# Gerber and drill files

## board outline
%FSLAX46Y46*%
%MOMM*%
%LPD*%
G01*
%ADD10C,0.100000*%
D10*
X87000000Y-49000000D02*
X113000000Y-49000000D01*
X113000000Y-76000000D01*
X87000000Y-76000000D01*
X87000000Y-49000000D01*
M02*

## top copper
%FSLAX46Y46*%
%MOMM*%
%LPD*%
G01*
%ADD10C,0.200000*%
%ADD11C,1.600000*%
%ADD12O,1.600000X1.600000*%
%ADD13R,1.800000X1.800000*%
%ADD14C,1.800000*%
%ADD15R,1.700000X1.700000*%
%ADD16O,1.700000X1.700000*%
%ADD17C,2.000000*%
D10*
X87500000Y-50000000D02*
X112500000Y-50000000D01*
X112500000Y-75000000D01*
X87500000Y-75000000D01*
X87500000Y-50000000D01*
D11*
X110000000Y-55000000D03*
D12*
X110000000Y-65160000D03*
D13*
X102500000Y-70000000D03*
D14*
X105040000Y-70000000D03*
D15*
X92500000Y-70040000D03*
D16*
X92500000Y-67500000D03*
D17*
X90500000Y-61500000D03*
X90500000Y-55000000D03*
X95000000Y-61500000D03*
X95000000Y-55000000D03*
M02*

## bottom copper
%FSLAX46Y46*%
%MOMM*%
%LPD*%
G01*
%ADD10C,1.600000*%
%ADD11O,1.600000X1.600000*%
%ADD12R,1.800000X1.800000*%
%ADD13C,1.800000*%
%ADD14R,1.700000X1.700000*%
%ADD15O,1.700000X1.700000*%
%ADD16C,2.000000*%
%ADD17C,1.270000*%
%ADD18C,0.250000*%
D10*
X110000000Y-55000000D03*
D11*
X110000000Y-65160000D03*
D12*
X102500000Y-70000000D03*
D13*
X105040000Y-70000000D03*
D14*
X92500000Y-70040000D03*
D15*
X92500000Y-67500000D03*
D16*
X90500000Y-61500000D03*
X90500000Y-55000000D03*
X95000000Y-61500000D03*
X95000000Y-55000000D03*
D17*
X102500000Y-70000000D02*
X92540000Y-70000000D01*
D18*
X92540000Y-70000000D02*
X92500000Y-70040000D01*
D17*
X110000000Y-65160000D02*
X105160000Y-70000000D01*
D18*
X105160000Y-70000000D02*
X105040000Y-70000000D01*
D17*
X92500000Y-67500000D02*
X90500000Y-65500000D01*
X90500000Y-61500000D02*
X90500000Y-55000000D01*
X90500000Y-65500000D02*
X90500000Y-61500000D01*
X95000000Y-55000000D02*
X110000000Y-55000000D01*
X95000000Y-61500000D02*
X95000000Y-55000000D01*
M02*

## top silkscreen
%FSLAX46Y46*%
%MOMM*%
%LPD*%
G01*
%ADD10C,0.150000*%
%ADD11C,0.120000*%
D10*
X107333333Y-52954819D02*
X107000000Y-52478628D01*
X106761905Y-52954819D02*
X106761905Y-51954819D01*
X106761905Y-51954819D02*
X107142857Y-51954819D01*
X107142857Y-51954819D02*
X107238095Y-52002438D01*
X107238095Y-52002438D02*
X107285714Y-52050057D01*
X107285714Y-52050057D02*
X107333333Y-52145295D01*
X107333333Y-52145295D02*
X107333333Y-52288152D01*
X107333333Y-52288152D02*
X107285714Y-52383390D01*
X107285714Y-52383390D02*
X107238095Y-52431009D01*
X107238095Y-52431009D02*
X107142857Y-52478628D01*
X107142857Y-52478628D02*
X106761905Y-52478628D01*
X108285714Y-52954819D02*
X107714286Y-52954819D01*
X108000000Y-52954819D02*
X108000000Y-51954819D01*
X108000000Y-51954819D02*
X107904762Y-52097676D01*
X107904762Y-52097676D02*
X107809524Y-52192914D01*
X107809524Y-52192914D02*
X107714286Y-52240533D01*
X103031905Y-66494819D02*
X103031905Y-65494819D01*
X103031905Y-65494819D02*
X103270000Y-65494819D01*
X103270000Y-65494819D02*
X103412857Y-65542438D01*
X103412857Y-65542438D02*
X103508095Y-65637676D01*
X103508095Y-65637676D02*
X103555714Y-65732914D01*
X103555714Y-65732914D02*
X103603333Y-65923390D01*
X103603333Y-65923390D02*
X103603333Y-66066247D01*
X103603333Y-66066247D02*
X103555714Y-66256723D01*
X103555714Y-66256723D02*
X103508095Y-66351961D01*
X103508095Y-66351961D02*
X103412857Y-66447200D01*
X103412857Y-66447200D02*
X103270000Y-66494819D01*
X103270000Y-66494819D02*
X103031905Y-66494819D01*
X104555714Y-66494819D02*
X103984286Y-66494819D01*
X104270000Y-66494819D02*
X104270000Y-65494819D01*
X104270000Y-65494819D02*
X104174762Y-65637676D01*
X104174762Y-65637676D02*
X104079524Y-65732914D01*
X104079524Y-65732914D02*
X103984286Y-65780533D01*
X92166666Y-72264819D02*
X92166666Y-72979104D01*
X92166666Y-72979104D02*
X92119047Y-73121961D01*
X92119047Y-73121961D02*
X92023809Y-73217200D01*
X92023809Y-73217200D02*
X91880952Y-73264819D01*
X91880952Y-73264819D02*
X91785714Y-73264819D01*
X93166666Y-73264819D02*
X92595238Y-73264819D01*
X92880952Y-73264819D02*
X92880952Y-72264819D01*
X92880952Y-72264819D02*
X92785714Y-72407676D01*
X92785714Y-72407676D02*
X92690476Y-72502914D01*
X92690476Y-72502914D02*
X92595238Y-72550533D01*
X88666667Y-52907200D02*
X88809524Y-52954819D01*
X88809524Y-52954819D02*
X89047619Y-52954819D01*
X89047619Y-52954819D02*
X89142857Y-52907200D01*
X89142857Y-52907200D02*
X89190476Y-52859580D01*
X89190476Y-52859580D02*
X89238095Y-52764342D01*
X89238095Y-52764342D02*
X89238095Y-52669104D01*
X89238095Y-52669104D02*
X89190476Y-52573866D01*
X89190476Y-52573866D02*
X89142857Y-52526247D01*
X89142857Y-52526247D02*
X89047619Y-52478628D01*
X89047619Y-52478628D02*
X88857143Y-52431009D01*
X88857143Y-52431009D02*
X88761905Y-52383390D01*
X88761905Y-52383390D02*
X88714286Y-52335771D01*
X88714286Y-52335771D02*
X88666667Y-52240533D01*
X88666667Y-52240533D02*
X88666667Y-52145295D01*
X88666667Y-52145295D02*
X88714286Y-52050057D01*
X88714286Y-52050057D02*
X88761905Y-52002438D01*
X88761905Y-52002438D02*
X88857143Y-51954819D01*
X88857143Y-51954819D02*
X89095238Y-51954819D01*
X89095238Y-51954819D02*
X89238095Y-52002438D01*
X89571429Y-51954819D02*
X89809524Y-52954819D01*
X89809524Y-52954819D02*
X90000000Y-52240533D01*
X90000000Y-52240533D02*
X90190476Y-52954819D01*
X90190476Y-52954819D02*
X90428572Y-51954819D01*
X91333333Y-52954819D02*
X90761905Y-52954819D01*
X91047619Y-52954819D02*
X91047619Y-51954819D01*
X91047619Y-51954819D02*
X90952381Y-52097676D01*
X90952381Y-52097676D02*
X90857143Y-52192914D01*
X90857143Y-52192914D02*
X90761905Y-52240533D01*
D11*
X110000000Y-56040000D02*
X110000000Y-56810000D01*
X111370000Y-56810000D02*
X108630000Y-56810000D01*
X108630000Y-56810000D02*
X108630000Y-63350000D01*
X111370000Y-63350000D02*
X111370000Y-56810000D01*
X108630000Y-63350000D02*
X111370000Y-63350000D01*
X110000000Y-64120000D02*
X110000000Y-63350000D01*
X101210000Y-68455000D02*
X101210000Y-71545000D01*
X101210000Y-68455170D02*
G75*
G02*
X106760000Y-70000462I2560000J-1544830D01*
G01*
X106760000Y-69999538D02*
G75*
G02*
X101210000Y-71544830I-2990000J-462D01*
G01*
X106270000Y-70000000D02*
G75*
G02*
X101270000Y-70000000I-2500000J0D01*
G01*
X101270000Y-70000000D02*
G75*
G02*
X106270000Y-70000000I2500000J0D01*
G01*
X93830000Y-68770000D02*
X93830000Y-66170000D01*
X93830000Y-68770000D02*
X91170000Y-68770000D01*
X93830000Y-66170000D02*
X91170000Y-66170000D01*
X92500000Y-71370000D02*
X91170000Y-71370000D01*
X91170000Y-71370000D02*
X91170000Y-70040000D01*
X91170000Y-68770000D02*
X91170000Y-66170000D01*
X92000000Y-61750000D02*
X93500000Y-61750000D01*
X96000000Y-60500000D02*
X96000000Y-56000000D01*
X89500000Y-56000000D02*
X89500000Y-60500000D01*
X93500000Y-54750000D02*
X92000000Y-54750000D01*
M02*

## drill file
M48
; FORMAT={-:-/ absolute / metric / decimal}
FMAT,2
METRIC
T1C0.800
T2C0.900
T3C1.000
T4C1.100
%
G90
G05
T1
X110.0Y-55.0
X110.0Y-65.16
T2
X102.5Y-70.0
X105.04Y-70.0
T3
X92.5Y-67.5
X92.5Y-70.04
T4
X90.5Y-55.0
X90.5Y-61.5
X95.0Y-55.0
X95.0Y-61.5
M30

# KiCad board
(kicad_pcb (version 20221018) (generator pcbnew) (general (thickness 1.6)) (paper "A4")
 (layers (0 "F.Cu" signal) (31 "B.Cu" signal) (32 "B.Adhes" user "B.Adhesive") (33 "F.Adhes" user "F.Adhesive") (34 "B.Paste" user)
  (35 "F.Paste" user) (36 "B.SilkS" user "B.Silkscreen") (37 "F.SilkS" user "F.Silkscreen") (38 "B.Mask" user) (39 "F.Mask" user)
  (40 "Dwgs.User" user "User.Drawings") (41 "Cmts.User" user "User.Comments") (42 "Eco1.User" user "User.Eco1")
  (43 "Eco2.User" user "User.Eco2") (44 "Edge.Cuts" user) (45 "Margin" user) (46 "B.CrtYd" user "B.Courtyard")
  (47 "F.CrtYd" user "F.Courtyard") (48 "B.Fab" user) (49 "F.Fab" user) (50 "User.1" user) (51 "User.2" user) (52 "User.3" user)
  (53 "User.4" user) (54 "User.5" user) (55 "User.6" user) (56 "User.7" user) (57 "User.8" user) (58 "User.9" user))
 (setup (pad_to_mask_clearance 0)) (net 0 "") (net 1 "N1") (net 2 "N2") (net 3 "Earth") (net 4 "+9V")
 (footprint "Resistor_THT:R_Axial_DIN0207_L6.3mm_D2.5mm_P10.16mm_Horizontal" (layer "F.Cu") (at 110 55 -90)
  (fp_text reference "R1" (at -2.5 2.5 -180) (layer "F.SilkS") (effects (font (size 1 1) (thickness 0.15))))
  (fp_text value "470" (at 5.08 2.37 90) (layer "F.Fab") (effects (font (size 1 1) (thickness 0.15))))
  (fp_line (start 1.04 0) (end 1.81 0) (stroke (width 0.12) (type solid)) (layer "F.SilkS"))
  (fp_line (start 1.81 -1.37) (end 1.81 1.37) (stroke (width 0.12) (type solid)) (layer "F.SilkS"))
  (fp_line (start 1.81 1.37) (end 8.35 1.37) (stroke (width 0.12) (type solid)) (layer "F.SilkS"))
  (fp_line (start 8.35 -1.37) (end 1.81 -1.37) (stroke (width 0.12) (type solid)) (layer "F.SilkS"))
  (fp_line (start 8.35 1.37) (end 8.35 -1.37) (stroke (width 0.12) (type solid)) (layer "F.SilkS"))
  (fp_line (start 9.12 0) (end 8.35 0) (stroke (width 0.12) (type solid)) (layer "F.SilkS"))
  (pad "1" thru_hole circle (at 0 0 270) (size 1.6 1.6) (drill 0.8) (layers "*.Cu" "*.Mask") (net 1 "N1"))
  (pad "2" thru_hole oval (at 10.16 0 270) (size 1.6 1.6) (drill 0.8) (layers "*.Cu" "*.Mask") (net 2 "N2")))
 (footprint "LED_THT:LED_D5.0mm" (layer "F.Cu") (at 102.5 70)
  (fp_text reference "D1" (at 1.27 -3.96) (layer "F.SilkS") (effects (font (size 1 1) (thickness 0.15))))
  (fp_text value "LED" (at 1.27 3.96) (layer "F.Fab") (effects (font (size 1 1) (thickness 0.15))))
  (fp_line (start -1.29 -1.545) (end -1.29 1.545) (stroke (width 0.12) (type solid)) (layer "F.SilkS"))
  (fp_arc (start -1.29 -1.54483) (mid 2.072002 -2.880433) (end 4.26 0.000462) (stroke (width 0.12) (type solid)) (layer "F.SilkS"))
  (fp_arc (start 4.26 -0.000462) (mid 2.072002 2.880433) (end -1.29 1.54483) (stroke (width 0.12) (type solid)) (layer "F.SilkS"))
  (fp_circle (center 1.27 0) (end 3.77 0) (stroke (width 0.12) (type solid)) (fill none) (layer "F.SilkS"))
  (pad "1" thru_hole rect (at 0 0) (size 1.8 1.8) (drill 0.9) (layers "*.Cu" "*.Mask") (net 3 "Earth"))
  (pad "2" thru_hole circle (at 2.54 0) (size 1.8 1.8) (drill 0.9) (layers "*.Cu" "*.Mask") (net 2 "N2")))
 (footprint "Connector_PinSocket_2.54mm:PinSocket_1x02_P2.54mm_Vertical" (layer "F.Cu") (at 92.5 70.04 180)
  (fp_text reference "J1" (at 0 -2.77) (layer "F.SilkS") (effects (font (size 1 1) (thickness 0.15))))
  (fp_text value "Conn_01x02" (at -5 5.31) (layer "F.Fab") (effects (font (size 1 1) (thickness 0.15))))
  (fp_line (start -1.33 1.27) (end -1.33 3.87) (stroke (width 0.12) (type solid)) (layer "F.SilkS"))
  (fp_line (start -1.33 1.27) (end 1.33 1.27) (stroke (width 0.12) (type solid)) (layer "F.SilkS"))
  (fp_line (start -1.33 3.87) (end 1.33 3.87) (stroke (width 0.12) (type solid)) (layer "F.SilkS"))
  (fp_line (start 0 -1.33) (end 1.33 -1.33) (stroke (width 0.12) (type solid)) (layer "F.SilkS"))
  (fp_line (start 1.33 -1.33) (end 1.33 0) (stroke (width 0.12) (type solid)) (layer "F.SilkS"))
  (fp_line (start 1.33 1.27) (end 1.33 3.87) (stroke (width 0.12) (type solid)) (layer "F.SilkS"))
  (pad "1" thru_hole rect (at 0 0 180) (size 1.7 1.7) (drill 1) (layers "*.Cu" "*.Mask") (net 3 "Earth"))
  (pad "2" thru_hole oval (at 0 2.54 180) (size 1.7 1.7) (drill 1) (layers "*.Cu" "*.Mask") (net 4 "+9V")))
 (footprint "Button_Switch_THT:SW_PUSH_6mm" (layer "F.Cu") (at 90.5 61.5 90)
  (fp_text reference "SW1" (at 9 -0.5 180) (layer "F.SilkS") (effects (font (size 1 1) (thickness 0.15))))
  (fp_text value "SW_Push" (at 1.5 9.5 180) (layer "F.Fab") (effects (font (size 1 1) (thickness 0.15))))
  (fp_line (start -0.25 1.5) (end -0.25 3) (stroke (width 0.12) (type solid)) (layer "F.SilkS"))
  (fp_line (start 1 5.5) (end 5.5 5.5) (stroke (width 0.12) (type solid)) (layer "F.SilkS"))
  (fp_line (start 5.5 -1) (end 1 -1) (stroke (width 0.12) (type solid)) (layer "F.SilkS"))
  (fp_line (start 6.75 3) (end 6.75 1.5) (stroke (width 0.12) (type solid)) (layer "F.SilkS"))
  (pad "1" thru_hole circle (at 0 0 180) (size 2 2) (drill 1.1) (layers "*.Cu" "*.Mask") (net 4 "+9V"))
  (pad "1" thru_hole circle (at 6.5 0 180) (size 2 2) (drill 1.1) (layers "*.Cu" "*.Mask") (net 4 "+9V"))
  (pad "2" thru_hole circle (at 0 4.5 180) (size 2 2) (drill 1.1) (layers "*.Cu" "*.Mask") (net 1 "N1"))
  (pad "2" thru_hole circle (at 6.5 4.5 180) (size 2 2) (drill 1.1) (layers "*.Cu" "*.Mask") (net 1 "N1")))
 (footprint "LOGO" (layer "B.Cu") (at 103.378 61.722 180)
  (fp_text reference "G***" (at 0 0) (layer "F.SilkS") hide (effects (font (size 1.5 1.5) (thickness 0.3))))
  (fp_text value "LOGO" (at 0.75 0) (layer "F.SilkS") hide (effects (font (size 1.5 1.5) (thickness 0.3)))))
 (gr_rect (start 87.5 50) (end 112.5 75) (stroke (width 0.2) (type default)) (fill none) (layer "F.Cu"))
 (gr_rect (start 87 49) (end 113 76) (stroke (width 0.1) (type default)) (fill none) (layer "Edge.Cuts"))
 (segment (start 102.5 70) (end 92.54 70) (width 1.27) (layer "B.Cu") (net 3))
 (segment (start 92.54 70) (end 92.5 70.04) (width 0.25) (layer "B.Cu") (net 3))
 (segment (start 110 65.16) (end 105.16 70) (width 1.27) (layer "B.Cu") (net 2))
 (segment (start 105.16 70) (end 105.04 70) (width 0.25) (layer "B.Cu") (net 2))
 (segment (start 92.5 67.5) (end 90.5 65.5) (width 1.27) (layer "B.Cu") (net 4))
 (segment (start 90.5 61.5) (end 90.5 55) (width 1.27) (layer "B.Cu") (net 4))
 (segment (start 90.5 65.5) (end 90.5 61.5) (width 1.27) (layer "B.Cu") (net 4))
 (segment (start 95 55) (end 110 55) (width 1.27) (layer "B.Cu") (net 1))
 (segment (start 95 61.5) (end 95 55) (width 1.27) (layer "B.Cu") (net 1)))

